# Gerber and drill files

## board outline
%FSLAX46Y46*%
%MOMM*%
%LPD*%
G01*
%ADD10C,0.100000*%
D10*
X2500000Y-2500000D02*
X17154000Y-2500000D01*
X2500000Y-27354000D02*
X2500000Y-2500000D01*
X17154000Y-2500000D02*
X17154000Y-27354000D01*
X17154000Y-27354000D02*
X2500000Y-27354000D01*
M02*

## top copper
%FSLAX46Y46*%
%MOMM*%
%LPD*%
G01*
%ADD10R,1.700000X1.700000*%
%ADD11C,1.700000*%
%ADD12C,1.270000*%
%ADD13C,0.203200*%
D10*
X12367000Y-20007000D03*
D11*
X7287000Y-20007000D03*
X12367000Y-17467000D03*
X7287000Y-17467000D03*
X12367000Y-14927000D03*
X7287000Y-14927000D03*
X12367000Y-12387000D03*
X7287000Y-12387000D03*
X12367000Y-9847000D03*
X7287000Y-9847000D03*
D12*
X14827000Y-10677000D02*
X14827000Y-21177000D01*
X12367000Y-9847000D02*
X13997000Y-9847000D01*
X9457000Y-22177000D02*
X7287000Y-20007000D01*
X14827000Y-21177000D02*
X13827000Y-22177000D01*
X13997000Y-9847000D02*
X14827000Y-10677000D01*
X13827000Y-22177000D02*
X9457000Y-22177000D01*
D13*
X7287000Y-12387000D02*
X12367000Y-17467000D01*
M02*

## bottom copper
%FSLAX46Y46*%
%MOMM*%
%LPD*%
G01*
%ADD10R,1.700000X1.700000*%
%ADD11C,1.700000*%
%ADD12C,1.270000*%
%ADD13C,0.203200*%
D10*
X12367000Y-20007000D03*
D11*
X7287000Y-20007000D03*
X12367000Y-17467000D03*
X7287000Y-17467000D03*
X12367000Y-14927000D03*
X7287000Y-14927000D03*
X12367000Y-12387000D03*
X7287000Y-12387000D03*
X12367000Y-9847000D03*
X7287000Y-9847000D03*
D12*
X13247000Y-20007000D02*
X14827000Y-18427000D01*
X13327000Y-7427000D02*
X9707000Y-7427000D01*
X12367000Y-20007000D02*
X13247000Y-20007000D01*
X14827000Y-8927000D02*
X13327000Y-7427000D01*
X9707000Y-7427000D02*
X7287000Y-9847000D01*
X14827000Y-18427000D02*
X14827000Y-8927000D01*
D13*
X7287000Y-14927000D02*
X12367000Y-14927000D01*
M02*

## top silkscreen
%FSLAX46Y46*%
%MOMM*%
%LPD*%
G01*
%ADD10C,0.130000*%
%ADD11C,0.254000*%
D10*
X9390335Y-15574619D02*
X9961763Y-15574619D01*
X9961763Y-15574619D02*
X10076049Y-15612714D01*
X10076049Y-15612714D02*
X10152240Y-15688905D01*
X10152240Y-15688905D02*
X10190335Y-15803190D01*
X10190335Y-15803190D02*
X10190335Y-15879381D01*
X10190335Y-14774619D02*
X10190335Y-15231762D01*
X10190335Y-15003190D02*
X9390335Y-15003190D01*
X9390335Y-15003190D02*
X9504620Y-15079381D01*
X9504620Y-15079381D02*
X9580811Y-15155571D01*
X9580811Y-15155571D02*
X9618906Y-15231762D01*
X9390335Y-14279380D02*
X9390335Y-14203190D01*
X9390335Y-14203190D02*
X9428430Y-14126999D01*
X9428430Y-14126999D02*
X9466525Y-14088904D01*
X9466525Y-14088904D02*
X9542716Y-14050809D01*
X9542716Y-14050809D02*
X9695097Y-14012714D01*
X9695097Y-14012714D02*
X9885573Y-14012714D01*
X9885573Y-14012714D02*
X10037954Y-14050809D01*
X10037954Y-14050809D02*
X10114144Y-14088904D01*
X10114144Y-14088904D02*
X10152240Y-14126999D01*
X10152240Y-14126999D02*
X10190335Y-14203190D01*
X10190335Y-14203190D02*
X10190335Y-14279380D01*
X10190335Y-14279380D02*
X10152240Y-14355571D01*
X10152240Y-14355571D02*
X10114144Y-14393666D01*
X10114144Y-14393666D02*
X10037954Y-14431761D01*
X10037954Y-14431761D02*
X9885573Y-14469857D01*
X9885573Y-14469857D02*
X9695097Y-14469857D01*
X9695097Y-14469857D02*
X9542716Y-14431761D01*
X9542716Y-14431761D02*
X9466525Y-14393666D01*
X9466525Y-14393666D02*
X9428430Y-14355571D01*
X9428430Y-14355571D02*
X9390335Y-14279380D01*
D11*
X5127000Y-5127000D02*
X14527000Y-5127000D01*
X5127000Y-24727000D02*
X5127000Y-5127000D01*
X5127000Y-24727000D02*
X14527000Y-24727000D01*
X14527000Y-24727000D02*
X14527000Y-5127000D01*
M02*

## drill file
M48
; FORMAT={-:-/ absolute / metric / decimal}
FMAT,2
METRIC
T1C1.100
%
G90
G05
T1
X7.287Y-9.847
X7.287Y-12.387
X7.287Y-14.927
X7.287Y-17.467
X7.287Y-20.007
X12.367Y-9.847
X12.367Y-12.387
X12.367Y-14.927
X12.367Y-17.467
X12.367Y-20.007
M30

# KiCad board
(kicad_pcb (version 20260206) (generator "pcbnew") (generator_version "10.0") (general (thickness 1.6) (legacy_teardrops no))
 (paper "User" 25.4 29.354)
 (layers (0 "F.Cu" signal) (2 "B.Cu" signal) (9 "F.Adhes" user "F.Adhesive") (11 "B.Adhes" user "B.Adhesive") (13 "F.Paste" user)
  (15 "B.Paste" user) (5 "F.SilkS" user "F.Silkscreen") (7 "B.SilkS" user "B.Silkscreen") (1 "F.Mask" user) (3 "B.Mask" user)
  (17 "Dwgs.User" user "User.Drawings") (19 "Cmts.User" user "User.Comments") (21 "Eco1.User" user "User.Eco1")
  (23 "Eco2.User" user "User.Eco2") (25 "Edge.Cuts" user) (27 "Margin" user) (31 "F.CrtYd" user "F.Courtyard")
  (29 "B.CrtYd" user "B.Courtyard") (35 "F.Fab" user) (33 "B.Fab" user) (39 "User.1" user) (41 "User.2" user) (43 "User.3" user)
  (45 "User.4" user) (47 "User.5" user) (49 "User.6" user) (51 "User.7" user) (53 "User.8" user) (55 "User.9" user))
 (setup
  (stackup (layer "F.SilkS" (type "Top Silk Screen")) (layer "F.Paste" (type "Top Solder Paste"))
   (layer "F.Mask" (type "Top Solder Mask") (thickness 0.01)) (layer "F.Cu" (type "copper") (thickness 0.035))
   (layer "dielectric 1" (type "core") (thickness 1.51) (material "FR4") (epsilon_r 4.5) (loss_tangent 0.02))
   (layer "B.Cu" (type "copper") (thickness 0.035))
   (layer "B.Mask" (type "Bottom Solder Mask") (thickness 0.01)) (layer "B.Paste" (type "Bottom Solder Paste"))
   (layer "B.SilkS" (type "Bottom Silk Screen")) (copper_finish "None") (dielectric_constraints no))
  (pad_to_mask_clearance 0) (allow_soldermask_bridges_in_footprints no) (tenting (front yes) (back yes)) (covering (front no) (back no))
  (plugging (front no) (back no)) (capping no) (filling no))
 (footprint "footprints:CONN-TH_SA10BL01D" (layer "F.Cu") (at 9.827 14.927 90)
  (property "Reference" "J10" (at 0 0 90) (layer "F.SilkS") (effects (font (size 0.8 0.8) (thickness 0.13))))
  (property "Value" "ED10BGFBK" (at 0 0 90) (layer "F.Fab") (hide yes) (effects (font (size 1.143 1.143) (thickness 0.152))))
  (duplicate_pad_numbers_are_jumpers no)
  (fp_line (start 9.8 -4.7) (end 9.8 4.7) (stroke (width 0.254) (type solid)) (layer "F.SilkS"))
  (fp_line (start -9.8 -4.7) (end 9.8 -4.7) (stroke (width 0.254) (type solid)) (layer "F.SilkS"))
  (fp_line (start -9.8 -4.7) (end -9.8 4.7) (stroke (width 0.254) (type solid)) (layer "F.SilkS"))
  (fp_line (start -9.8 4.7) (end 9.8 4.7) (stroke (width 0.254) (type solid)) (layer "F.SilkS"))
  (pad "1" thru_hole rect (at -5.08 2.54 90) (size 1.7 1.7) (drill 1.1) (layers "*.Cu" "*.Paste" "*.Mask") (remove_unused_layers no)
   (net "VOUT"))
  (pad "2" thru_hole circle (at -5.08 -2.54 90) (size 1.7 1.7) (drill 1.1) (layers "*.Cu" "*.Paste" "*.Mask") (remove_unused_layers no)
   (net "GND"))
  (pad "3" thru_hole circle (at -2.54 2.54 90) (size 1.7 1.7) (drill 1.1) (layers "*.Cu" "*.Paste" "*.Mask") (remove_unused_layers no)
   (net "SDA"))
  (pad "4" thru_hole circle (at -2.54 -2.54 90) (size 1.7 1.7) (drill 1.1) (layers "*.Cu" "*.Paste" "*.Mask") (remove_unused_layers no)
   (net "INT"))
  (pad "5" thru_hole circle (at 0 2.54 90) (size 1.7 1.7) (drill 1.1) (layers "*.Cu" "*.Paste" "*.Mask") (remove_unused_layers no)
   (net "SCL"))
  (pad "6" thru_hole circle (at 0 -2.54 90) (size 1.7 1.7) (drill 1.1) (layers "*.Cu" "*.Paste" "*.Mask") (remove_unused_layers no)
   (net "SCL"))
  (pad "7" thru_hole circle (at 2.54 2.54 90) (size 1.7 1.7) (drill 1.1) (layers "*.Cu" "*.Paste" "*.Mask") (remove_unused_layers no)
   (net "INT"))
  (pad "8" thru_hole circle (at 2.54 -2.54 90) (size 1.7 1.7) (drill 1.1) (layers "*.Cu" "*.Paste" "*.Mask") (remove_unused_layers no)
   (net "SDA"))
  (pad "9" thru_hole circle (at 5.08 2.54 90) (size 1.7 1.7) (drill 1.1) (layers "*.Cu" "*.Paste" "*.Mask") (remove_unused_layers no)
   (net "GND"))
  (pad "10" thru_hole circle (at 5.08 -2.54 90) (size 1.7 1.7) (drill 1.1) (layers "*.Cu" "*.Paste" "*.Mask") (remove_unused_layers no)
   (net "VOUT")))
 (gr_line (start 2.5 2.5) (end 17.154 2.5) (stroke (width 0.1) (type default)) (layer "Edge.Cuts"))
 (gr_line (start 2.5 27.354) (end 2.5 2.5) (stroke (width 0.1) (type default)) (layer "Edge.Cuts"))
 (gr_line (start 17.154 2.5) (end 17.154 27.354) (stroke (width 0.1) (type default)) (layer "Edge.Cuts"))
 (gr_line (start 17.154 27.354) (end 2.5 27.354) (stroke (width 0.1) (type default)) (layer "Edge.Cuts"))
 (segment (start 13.247 20.007) (end 14.827 18.427) (width 1.27) (layer "B.Cu") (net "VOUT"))
 (segment (start 13.327 7.427) (end 9.707 7.427) (width 1.27) (layer "B.Cu") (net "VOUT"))
 (segment (start 12.367 20.007) (end 13.247 20.007) (width 1.27) (layer "B.Cu") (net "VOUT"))
 (segment (start 14.827 8.927) (end 13.327 7.427) (width 1.27) (layer "B.Cu") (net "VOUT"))
 (segment (start 9.707 7.427) (end 7.287 9.847) (width 1.27) (layer "B.Cu") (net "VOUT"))
 (segment (start 14.827 18.427) (end 14.827 8.927) (width 1.27) (layer "B.Cu") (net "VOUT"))
 (segment (start 14.827 10.677) (end 14.827 21.177) (width 1.27) (layer "F.Cu") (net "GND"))
 (segment (start 12.367 9.847) (end 13.997 9.847) (width 1.27) (layer "F.Cu") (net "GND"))
 (segment (start 9.457 22.177) (end 7.287 20.007) (width 1.27) (layer "F.Cu") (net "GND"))
 (segment (start 14.827 21.177) (end 13.827 22.177) (width 1.27) (layer "F.Cu") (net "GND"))
 (segment (start 13.997 9.847) (end 14.827 10.677) (width 1.27) (layer "F.Cu") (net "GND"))
 (segment (start 13.827 22.177) (end 9.457 22.177) (width 1.27) (layer "F.Cu") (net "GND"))
 (segment (start 7.287 12.387) (end 12.367 17.467) (width 0.2032) (layer "F.Cu") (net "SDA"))
 (segment (start 7.287 14.927) (end 12.367 14.927) (width 0.2032) (layer "B.Cu") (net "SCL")))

